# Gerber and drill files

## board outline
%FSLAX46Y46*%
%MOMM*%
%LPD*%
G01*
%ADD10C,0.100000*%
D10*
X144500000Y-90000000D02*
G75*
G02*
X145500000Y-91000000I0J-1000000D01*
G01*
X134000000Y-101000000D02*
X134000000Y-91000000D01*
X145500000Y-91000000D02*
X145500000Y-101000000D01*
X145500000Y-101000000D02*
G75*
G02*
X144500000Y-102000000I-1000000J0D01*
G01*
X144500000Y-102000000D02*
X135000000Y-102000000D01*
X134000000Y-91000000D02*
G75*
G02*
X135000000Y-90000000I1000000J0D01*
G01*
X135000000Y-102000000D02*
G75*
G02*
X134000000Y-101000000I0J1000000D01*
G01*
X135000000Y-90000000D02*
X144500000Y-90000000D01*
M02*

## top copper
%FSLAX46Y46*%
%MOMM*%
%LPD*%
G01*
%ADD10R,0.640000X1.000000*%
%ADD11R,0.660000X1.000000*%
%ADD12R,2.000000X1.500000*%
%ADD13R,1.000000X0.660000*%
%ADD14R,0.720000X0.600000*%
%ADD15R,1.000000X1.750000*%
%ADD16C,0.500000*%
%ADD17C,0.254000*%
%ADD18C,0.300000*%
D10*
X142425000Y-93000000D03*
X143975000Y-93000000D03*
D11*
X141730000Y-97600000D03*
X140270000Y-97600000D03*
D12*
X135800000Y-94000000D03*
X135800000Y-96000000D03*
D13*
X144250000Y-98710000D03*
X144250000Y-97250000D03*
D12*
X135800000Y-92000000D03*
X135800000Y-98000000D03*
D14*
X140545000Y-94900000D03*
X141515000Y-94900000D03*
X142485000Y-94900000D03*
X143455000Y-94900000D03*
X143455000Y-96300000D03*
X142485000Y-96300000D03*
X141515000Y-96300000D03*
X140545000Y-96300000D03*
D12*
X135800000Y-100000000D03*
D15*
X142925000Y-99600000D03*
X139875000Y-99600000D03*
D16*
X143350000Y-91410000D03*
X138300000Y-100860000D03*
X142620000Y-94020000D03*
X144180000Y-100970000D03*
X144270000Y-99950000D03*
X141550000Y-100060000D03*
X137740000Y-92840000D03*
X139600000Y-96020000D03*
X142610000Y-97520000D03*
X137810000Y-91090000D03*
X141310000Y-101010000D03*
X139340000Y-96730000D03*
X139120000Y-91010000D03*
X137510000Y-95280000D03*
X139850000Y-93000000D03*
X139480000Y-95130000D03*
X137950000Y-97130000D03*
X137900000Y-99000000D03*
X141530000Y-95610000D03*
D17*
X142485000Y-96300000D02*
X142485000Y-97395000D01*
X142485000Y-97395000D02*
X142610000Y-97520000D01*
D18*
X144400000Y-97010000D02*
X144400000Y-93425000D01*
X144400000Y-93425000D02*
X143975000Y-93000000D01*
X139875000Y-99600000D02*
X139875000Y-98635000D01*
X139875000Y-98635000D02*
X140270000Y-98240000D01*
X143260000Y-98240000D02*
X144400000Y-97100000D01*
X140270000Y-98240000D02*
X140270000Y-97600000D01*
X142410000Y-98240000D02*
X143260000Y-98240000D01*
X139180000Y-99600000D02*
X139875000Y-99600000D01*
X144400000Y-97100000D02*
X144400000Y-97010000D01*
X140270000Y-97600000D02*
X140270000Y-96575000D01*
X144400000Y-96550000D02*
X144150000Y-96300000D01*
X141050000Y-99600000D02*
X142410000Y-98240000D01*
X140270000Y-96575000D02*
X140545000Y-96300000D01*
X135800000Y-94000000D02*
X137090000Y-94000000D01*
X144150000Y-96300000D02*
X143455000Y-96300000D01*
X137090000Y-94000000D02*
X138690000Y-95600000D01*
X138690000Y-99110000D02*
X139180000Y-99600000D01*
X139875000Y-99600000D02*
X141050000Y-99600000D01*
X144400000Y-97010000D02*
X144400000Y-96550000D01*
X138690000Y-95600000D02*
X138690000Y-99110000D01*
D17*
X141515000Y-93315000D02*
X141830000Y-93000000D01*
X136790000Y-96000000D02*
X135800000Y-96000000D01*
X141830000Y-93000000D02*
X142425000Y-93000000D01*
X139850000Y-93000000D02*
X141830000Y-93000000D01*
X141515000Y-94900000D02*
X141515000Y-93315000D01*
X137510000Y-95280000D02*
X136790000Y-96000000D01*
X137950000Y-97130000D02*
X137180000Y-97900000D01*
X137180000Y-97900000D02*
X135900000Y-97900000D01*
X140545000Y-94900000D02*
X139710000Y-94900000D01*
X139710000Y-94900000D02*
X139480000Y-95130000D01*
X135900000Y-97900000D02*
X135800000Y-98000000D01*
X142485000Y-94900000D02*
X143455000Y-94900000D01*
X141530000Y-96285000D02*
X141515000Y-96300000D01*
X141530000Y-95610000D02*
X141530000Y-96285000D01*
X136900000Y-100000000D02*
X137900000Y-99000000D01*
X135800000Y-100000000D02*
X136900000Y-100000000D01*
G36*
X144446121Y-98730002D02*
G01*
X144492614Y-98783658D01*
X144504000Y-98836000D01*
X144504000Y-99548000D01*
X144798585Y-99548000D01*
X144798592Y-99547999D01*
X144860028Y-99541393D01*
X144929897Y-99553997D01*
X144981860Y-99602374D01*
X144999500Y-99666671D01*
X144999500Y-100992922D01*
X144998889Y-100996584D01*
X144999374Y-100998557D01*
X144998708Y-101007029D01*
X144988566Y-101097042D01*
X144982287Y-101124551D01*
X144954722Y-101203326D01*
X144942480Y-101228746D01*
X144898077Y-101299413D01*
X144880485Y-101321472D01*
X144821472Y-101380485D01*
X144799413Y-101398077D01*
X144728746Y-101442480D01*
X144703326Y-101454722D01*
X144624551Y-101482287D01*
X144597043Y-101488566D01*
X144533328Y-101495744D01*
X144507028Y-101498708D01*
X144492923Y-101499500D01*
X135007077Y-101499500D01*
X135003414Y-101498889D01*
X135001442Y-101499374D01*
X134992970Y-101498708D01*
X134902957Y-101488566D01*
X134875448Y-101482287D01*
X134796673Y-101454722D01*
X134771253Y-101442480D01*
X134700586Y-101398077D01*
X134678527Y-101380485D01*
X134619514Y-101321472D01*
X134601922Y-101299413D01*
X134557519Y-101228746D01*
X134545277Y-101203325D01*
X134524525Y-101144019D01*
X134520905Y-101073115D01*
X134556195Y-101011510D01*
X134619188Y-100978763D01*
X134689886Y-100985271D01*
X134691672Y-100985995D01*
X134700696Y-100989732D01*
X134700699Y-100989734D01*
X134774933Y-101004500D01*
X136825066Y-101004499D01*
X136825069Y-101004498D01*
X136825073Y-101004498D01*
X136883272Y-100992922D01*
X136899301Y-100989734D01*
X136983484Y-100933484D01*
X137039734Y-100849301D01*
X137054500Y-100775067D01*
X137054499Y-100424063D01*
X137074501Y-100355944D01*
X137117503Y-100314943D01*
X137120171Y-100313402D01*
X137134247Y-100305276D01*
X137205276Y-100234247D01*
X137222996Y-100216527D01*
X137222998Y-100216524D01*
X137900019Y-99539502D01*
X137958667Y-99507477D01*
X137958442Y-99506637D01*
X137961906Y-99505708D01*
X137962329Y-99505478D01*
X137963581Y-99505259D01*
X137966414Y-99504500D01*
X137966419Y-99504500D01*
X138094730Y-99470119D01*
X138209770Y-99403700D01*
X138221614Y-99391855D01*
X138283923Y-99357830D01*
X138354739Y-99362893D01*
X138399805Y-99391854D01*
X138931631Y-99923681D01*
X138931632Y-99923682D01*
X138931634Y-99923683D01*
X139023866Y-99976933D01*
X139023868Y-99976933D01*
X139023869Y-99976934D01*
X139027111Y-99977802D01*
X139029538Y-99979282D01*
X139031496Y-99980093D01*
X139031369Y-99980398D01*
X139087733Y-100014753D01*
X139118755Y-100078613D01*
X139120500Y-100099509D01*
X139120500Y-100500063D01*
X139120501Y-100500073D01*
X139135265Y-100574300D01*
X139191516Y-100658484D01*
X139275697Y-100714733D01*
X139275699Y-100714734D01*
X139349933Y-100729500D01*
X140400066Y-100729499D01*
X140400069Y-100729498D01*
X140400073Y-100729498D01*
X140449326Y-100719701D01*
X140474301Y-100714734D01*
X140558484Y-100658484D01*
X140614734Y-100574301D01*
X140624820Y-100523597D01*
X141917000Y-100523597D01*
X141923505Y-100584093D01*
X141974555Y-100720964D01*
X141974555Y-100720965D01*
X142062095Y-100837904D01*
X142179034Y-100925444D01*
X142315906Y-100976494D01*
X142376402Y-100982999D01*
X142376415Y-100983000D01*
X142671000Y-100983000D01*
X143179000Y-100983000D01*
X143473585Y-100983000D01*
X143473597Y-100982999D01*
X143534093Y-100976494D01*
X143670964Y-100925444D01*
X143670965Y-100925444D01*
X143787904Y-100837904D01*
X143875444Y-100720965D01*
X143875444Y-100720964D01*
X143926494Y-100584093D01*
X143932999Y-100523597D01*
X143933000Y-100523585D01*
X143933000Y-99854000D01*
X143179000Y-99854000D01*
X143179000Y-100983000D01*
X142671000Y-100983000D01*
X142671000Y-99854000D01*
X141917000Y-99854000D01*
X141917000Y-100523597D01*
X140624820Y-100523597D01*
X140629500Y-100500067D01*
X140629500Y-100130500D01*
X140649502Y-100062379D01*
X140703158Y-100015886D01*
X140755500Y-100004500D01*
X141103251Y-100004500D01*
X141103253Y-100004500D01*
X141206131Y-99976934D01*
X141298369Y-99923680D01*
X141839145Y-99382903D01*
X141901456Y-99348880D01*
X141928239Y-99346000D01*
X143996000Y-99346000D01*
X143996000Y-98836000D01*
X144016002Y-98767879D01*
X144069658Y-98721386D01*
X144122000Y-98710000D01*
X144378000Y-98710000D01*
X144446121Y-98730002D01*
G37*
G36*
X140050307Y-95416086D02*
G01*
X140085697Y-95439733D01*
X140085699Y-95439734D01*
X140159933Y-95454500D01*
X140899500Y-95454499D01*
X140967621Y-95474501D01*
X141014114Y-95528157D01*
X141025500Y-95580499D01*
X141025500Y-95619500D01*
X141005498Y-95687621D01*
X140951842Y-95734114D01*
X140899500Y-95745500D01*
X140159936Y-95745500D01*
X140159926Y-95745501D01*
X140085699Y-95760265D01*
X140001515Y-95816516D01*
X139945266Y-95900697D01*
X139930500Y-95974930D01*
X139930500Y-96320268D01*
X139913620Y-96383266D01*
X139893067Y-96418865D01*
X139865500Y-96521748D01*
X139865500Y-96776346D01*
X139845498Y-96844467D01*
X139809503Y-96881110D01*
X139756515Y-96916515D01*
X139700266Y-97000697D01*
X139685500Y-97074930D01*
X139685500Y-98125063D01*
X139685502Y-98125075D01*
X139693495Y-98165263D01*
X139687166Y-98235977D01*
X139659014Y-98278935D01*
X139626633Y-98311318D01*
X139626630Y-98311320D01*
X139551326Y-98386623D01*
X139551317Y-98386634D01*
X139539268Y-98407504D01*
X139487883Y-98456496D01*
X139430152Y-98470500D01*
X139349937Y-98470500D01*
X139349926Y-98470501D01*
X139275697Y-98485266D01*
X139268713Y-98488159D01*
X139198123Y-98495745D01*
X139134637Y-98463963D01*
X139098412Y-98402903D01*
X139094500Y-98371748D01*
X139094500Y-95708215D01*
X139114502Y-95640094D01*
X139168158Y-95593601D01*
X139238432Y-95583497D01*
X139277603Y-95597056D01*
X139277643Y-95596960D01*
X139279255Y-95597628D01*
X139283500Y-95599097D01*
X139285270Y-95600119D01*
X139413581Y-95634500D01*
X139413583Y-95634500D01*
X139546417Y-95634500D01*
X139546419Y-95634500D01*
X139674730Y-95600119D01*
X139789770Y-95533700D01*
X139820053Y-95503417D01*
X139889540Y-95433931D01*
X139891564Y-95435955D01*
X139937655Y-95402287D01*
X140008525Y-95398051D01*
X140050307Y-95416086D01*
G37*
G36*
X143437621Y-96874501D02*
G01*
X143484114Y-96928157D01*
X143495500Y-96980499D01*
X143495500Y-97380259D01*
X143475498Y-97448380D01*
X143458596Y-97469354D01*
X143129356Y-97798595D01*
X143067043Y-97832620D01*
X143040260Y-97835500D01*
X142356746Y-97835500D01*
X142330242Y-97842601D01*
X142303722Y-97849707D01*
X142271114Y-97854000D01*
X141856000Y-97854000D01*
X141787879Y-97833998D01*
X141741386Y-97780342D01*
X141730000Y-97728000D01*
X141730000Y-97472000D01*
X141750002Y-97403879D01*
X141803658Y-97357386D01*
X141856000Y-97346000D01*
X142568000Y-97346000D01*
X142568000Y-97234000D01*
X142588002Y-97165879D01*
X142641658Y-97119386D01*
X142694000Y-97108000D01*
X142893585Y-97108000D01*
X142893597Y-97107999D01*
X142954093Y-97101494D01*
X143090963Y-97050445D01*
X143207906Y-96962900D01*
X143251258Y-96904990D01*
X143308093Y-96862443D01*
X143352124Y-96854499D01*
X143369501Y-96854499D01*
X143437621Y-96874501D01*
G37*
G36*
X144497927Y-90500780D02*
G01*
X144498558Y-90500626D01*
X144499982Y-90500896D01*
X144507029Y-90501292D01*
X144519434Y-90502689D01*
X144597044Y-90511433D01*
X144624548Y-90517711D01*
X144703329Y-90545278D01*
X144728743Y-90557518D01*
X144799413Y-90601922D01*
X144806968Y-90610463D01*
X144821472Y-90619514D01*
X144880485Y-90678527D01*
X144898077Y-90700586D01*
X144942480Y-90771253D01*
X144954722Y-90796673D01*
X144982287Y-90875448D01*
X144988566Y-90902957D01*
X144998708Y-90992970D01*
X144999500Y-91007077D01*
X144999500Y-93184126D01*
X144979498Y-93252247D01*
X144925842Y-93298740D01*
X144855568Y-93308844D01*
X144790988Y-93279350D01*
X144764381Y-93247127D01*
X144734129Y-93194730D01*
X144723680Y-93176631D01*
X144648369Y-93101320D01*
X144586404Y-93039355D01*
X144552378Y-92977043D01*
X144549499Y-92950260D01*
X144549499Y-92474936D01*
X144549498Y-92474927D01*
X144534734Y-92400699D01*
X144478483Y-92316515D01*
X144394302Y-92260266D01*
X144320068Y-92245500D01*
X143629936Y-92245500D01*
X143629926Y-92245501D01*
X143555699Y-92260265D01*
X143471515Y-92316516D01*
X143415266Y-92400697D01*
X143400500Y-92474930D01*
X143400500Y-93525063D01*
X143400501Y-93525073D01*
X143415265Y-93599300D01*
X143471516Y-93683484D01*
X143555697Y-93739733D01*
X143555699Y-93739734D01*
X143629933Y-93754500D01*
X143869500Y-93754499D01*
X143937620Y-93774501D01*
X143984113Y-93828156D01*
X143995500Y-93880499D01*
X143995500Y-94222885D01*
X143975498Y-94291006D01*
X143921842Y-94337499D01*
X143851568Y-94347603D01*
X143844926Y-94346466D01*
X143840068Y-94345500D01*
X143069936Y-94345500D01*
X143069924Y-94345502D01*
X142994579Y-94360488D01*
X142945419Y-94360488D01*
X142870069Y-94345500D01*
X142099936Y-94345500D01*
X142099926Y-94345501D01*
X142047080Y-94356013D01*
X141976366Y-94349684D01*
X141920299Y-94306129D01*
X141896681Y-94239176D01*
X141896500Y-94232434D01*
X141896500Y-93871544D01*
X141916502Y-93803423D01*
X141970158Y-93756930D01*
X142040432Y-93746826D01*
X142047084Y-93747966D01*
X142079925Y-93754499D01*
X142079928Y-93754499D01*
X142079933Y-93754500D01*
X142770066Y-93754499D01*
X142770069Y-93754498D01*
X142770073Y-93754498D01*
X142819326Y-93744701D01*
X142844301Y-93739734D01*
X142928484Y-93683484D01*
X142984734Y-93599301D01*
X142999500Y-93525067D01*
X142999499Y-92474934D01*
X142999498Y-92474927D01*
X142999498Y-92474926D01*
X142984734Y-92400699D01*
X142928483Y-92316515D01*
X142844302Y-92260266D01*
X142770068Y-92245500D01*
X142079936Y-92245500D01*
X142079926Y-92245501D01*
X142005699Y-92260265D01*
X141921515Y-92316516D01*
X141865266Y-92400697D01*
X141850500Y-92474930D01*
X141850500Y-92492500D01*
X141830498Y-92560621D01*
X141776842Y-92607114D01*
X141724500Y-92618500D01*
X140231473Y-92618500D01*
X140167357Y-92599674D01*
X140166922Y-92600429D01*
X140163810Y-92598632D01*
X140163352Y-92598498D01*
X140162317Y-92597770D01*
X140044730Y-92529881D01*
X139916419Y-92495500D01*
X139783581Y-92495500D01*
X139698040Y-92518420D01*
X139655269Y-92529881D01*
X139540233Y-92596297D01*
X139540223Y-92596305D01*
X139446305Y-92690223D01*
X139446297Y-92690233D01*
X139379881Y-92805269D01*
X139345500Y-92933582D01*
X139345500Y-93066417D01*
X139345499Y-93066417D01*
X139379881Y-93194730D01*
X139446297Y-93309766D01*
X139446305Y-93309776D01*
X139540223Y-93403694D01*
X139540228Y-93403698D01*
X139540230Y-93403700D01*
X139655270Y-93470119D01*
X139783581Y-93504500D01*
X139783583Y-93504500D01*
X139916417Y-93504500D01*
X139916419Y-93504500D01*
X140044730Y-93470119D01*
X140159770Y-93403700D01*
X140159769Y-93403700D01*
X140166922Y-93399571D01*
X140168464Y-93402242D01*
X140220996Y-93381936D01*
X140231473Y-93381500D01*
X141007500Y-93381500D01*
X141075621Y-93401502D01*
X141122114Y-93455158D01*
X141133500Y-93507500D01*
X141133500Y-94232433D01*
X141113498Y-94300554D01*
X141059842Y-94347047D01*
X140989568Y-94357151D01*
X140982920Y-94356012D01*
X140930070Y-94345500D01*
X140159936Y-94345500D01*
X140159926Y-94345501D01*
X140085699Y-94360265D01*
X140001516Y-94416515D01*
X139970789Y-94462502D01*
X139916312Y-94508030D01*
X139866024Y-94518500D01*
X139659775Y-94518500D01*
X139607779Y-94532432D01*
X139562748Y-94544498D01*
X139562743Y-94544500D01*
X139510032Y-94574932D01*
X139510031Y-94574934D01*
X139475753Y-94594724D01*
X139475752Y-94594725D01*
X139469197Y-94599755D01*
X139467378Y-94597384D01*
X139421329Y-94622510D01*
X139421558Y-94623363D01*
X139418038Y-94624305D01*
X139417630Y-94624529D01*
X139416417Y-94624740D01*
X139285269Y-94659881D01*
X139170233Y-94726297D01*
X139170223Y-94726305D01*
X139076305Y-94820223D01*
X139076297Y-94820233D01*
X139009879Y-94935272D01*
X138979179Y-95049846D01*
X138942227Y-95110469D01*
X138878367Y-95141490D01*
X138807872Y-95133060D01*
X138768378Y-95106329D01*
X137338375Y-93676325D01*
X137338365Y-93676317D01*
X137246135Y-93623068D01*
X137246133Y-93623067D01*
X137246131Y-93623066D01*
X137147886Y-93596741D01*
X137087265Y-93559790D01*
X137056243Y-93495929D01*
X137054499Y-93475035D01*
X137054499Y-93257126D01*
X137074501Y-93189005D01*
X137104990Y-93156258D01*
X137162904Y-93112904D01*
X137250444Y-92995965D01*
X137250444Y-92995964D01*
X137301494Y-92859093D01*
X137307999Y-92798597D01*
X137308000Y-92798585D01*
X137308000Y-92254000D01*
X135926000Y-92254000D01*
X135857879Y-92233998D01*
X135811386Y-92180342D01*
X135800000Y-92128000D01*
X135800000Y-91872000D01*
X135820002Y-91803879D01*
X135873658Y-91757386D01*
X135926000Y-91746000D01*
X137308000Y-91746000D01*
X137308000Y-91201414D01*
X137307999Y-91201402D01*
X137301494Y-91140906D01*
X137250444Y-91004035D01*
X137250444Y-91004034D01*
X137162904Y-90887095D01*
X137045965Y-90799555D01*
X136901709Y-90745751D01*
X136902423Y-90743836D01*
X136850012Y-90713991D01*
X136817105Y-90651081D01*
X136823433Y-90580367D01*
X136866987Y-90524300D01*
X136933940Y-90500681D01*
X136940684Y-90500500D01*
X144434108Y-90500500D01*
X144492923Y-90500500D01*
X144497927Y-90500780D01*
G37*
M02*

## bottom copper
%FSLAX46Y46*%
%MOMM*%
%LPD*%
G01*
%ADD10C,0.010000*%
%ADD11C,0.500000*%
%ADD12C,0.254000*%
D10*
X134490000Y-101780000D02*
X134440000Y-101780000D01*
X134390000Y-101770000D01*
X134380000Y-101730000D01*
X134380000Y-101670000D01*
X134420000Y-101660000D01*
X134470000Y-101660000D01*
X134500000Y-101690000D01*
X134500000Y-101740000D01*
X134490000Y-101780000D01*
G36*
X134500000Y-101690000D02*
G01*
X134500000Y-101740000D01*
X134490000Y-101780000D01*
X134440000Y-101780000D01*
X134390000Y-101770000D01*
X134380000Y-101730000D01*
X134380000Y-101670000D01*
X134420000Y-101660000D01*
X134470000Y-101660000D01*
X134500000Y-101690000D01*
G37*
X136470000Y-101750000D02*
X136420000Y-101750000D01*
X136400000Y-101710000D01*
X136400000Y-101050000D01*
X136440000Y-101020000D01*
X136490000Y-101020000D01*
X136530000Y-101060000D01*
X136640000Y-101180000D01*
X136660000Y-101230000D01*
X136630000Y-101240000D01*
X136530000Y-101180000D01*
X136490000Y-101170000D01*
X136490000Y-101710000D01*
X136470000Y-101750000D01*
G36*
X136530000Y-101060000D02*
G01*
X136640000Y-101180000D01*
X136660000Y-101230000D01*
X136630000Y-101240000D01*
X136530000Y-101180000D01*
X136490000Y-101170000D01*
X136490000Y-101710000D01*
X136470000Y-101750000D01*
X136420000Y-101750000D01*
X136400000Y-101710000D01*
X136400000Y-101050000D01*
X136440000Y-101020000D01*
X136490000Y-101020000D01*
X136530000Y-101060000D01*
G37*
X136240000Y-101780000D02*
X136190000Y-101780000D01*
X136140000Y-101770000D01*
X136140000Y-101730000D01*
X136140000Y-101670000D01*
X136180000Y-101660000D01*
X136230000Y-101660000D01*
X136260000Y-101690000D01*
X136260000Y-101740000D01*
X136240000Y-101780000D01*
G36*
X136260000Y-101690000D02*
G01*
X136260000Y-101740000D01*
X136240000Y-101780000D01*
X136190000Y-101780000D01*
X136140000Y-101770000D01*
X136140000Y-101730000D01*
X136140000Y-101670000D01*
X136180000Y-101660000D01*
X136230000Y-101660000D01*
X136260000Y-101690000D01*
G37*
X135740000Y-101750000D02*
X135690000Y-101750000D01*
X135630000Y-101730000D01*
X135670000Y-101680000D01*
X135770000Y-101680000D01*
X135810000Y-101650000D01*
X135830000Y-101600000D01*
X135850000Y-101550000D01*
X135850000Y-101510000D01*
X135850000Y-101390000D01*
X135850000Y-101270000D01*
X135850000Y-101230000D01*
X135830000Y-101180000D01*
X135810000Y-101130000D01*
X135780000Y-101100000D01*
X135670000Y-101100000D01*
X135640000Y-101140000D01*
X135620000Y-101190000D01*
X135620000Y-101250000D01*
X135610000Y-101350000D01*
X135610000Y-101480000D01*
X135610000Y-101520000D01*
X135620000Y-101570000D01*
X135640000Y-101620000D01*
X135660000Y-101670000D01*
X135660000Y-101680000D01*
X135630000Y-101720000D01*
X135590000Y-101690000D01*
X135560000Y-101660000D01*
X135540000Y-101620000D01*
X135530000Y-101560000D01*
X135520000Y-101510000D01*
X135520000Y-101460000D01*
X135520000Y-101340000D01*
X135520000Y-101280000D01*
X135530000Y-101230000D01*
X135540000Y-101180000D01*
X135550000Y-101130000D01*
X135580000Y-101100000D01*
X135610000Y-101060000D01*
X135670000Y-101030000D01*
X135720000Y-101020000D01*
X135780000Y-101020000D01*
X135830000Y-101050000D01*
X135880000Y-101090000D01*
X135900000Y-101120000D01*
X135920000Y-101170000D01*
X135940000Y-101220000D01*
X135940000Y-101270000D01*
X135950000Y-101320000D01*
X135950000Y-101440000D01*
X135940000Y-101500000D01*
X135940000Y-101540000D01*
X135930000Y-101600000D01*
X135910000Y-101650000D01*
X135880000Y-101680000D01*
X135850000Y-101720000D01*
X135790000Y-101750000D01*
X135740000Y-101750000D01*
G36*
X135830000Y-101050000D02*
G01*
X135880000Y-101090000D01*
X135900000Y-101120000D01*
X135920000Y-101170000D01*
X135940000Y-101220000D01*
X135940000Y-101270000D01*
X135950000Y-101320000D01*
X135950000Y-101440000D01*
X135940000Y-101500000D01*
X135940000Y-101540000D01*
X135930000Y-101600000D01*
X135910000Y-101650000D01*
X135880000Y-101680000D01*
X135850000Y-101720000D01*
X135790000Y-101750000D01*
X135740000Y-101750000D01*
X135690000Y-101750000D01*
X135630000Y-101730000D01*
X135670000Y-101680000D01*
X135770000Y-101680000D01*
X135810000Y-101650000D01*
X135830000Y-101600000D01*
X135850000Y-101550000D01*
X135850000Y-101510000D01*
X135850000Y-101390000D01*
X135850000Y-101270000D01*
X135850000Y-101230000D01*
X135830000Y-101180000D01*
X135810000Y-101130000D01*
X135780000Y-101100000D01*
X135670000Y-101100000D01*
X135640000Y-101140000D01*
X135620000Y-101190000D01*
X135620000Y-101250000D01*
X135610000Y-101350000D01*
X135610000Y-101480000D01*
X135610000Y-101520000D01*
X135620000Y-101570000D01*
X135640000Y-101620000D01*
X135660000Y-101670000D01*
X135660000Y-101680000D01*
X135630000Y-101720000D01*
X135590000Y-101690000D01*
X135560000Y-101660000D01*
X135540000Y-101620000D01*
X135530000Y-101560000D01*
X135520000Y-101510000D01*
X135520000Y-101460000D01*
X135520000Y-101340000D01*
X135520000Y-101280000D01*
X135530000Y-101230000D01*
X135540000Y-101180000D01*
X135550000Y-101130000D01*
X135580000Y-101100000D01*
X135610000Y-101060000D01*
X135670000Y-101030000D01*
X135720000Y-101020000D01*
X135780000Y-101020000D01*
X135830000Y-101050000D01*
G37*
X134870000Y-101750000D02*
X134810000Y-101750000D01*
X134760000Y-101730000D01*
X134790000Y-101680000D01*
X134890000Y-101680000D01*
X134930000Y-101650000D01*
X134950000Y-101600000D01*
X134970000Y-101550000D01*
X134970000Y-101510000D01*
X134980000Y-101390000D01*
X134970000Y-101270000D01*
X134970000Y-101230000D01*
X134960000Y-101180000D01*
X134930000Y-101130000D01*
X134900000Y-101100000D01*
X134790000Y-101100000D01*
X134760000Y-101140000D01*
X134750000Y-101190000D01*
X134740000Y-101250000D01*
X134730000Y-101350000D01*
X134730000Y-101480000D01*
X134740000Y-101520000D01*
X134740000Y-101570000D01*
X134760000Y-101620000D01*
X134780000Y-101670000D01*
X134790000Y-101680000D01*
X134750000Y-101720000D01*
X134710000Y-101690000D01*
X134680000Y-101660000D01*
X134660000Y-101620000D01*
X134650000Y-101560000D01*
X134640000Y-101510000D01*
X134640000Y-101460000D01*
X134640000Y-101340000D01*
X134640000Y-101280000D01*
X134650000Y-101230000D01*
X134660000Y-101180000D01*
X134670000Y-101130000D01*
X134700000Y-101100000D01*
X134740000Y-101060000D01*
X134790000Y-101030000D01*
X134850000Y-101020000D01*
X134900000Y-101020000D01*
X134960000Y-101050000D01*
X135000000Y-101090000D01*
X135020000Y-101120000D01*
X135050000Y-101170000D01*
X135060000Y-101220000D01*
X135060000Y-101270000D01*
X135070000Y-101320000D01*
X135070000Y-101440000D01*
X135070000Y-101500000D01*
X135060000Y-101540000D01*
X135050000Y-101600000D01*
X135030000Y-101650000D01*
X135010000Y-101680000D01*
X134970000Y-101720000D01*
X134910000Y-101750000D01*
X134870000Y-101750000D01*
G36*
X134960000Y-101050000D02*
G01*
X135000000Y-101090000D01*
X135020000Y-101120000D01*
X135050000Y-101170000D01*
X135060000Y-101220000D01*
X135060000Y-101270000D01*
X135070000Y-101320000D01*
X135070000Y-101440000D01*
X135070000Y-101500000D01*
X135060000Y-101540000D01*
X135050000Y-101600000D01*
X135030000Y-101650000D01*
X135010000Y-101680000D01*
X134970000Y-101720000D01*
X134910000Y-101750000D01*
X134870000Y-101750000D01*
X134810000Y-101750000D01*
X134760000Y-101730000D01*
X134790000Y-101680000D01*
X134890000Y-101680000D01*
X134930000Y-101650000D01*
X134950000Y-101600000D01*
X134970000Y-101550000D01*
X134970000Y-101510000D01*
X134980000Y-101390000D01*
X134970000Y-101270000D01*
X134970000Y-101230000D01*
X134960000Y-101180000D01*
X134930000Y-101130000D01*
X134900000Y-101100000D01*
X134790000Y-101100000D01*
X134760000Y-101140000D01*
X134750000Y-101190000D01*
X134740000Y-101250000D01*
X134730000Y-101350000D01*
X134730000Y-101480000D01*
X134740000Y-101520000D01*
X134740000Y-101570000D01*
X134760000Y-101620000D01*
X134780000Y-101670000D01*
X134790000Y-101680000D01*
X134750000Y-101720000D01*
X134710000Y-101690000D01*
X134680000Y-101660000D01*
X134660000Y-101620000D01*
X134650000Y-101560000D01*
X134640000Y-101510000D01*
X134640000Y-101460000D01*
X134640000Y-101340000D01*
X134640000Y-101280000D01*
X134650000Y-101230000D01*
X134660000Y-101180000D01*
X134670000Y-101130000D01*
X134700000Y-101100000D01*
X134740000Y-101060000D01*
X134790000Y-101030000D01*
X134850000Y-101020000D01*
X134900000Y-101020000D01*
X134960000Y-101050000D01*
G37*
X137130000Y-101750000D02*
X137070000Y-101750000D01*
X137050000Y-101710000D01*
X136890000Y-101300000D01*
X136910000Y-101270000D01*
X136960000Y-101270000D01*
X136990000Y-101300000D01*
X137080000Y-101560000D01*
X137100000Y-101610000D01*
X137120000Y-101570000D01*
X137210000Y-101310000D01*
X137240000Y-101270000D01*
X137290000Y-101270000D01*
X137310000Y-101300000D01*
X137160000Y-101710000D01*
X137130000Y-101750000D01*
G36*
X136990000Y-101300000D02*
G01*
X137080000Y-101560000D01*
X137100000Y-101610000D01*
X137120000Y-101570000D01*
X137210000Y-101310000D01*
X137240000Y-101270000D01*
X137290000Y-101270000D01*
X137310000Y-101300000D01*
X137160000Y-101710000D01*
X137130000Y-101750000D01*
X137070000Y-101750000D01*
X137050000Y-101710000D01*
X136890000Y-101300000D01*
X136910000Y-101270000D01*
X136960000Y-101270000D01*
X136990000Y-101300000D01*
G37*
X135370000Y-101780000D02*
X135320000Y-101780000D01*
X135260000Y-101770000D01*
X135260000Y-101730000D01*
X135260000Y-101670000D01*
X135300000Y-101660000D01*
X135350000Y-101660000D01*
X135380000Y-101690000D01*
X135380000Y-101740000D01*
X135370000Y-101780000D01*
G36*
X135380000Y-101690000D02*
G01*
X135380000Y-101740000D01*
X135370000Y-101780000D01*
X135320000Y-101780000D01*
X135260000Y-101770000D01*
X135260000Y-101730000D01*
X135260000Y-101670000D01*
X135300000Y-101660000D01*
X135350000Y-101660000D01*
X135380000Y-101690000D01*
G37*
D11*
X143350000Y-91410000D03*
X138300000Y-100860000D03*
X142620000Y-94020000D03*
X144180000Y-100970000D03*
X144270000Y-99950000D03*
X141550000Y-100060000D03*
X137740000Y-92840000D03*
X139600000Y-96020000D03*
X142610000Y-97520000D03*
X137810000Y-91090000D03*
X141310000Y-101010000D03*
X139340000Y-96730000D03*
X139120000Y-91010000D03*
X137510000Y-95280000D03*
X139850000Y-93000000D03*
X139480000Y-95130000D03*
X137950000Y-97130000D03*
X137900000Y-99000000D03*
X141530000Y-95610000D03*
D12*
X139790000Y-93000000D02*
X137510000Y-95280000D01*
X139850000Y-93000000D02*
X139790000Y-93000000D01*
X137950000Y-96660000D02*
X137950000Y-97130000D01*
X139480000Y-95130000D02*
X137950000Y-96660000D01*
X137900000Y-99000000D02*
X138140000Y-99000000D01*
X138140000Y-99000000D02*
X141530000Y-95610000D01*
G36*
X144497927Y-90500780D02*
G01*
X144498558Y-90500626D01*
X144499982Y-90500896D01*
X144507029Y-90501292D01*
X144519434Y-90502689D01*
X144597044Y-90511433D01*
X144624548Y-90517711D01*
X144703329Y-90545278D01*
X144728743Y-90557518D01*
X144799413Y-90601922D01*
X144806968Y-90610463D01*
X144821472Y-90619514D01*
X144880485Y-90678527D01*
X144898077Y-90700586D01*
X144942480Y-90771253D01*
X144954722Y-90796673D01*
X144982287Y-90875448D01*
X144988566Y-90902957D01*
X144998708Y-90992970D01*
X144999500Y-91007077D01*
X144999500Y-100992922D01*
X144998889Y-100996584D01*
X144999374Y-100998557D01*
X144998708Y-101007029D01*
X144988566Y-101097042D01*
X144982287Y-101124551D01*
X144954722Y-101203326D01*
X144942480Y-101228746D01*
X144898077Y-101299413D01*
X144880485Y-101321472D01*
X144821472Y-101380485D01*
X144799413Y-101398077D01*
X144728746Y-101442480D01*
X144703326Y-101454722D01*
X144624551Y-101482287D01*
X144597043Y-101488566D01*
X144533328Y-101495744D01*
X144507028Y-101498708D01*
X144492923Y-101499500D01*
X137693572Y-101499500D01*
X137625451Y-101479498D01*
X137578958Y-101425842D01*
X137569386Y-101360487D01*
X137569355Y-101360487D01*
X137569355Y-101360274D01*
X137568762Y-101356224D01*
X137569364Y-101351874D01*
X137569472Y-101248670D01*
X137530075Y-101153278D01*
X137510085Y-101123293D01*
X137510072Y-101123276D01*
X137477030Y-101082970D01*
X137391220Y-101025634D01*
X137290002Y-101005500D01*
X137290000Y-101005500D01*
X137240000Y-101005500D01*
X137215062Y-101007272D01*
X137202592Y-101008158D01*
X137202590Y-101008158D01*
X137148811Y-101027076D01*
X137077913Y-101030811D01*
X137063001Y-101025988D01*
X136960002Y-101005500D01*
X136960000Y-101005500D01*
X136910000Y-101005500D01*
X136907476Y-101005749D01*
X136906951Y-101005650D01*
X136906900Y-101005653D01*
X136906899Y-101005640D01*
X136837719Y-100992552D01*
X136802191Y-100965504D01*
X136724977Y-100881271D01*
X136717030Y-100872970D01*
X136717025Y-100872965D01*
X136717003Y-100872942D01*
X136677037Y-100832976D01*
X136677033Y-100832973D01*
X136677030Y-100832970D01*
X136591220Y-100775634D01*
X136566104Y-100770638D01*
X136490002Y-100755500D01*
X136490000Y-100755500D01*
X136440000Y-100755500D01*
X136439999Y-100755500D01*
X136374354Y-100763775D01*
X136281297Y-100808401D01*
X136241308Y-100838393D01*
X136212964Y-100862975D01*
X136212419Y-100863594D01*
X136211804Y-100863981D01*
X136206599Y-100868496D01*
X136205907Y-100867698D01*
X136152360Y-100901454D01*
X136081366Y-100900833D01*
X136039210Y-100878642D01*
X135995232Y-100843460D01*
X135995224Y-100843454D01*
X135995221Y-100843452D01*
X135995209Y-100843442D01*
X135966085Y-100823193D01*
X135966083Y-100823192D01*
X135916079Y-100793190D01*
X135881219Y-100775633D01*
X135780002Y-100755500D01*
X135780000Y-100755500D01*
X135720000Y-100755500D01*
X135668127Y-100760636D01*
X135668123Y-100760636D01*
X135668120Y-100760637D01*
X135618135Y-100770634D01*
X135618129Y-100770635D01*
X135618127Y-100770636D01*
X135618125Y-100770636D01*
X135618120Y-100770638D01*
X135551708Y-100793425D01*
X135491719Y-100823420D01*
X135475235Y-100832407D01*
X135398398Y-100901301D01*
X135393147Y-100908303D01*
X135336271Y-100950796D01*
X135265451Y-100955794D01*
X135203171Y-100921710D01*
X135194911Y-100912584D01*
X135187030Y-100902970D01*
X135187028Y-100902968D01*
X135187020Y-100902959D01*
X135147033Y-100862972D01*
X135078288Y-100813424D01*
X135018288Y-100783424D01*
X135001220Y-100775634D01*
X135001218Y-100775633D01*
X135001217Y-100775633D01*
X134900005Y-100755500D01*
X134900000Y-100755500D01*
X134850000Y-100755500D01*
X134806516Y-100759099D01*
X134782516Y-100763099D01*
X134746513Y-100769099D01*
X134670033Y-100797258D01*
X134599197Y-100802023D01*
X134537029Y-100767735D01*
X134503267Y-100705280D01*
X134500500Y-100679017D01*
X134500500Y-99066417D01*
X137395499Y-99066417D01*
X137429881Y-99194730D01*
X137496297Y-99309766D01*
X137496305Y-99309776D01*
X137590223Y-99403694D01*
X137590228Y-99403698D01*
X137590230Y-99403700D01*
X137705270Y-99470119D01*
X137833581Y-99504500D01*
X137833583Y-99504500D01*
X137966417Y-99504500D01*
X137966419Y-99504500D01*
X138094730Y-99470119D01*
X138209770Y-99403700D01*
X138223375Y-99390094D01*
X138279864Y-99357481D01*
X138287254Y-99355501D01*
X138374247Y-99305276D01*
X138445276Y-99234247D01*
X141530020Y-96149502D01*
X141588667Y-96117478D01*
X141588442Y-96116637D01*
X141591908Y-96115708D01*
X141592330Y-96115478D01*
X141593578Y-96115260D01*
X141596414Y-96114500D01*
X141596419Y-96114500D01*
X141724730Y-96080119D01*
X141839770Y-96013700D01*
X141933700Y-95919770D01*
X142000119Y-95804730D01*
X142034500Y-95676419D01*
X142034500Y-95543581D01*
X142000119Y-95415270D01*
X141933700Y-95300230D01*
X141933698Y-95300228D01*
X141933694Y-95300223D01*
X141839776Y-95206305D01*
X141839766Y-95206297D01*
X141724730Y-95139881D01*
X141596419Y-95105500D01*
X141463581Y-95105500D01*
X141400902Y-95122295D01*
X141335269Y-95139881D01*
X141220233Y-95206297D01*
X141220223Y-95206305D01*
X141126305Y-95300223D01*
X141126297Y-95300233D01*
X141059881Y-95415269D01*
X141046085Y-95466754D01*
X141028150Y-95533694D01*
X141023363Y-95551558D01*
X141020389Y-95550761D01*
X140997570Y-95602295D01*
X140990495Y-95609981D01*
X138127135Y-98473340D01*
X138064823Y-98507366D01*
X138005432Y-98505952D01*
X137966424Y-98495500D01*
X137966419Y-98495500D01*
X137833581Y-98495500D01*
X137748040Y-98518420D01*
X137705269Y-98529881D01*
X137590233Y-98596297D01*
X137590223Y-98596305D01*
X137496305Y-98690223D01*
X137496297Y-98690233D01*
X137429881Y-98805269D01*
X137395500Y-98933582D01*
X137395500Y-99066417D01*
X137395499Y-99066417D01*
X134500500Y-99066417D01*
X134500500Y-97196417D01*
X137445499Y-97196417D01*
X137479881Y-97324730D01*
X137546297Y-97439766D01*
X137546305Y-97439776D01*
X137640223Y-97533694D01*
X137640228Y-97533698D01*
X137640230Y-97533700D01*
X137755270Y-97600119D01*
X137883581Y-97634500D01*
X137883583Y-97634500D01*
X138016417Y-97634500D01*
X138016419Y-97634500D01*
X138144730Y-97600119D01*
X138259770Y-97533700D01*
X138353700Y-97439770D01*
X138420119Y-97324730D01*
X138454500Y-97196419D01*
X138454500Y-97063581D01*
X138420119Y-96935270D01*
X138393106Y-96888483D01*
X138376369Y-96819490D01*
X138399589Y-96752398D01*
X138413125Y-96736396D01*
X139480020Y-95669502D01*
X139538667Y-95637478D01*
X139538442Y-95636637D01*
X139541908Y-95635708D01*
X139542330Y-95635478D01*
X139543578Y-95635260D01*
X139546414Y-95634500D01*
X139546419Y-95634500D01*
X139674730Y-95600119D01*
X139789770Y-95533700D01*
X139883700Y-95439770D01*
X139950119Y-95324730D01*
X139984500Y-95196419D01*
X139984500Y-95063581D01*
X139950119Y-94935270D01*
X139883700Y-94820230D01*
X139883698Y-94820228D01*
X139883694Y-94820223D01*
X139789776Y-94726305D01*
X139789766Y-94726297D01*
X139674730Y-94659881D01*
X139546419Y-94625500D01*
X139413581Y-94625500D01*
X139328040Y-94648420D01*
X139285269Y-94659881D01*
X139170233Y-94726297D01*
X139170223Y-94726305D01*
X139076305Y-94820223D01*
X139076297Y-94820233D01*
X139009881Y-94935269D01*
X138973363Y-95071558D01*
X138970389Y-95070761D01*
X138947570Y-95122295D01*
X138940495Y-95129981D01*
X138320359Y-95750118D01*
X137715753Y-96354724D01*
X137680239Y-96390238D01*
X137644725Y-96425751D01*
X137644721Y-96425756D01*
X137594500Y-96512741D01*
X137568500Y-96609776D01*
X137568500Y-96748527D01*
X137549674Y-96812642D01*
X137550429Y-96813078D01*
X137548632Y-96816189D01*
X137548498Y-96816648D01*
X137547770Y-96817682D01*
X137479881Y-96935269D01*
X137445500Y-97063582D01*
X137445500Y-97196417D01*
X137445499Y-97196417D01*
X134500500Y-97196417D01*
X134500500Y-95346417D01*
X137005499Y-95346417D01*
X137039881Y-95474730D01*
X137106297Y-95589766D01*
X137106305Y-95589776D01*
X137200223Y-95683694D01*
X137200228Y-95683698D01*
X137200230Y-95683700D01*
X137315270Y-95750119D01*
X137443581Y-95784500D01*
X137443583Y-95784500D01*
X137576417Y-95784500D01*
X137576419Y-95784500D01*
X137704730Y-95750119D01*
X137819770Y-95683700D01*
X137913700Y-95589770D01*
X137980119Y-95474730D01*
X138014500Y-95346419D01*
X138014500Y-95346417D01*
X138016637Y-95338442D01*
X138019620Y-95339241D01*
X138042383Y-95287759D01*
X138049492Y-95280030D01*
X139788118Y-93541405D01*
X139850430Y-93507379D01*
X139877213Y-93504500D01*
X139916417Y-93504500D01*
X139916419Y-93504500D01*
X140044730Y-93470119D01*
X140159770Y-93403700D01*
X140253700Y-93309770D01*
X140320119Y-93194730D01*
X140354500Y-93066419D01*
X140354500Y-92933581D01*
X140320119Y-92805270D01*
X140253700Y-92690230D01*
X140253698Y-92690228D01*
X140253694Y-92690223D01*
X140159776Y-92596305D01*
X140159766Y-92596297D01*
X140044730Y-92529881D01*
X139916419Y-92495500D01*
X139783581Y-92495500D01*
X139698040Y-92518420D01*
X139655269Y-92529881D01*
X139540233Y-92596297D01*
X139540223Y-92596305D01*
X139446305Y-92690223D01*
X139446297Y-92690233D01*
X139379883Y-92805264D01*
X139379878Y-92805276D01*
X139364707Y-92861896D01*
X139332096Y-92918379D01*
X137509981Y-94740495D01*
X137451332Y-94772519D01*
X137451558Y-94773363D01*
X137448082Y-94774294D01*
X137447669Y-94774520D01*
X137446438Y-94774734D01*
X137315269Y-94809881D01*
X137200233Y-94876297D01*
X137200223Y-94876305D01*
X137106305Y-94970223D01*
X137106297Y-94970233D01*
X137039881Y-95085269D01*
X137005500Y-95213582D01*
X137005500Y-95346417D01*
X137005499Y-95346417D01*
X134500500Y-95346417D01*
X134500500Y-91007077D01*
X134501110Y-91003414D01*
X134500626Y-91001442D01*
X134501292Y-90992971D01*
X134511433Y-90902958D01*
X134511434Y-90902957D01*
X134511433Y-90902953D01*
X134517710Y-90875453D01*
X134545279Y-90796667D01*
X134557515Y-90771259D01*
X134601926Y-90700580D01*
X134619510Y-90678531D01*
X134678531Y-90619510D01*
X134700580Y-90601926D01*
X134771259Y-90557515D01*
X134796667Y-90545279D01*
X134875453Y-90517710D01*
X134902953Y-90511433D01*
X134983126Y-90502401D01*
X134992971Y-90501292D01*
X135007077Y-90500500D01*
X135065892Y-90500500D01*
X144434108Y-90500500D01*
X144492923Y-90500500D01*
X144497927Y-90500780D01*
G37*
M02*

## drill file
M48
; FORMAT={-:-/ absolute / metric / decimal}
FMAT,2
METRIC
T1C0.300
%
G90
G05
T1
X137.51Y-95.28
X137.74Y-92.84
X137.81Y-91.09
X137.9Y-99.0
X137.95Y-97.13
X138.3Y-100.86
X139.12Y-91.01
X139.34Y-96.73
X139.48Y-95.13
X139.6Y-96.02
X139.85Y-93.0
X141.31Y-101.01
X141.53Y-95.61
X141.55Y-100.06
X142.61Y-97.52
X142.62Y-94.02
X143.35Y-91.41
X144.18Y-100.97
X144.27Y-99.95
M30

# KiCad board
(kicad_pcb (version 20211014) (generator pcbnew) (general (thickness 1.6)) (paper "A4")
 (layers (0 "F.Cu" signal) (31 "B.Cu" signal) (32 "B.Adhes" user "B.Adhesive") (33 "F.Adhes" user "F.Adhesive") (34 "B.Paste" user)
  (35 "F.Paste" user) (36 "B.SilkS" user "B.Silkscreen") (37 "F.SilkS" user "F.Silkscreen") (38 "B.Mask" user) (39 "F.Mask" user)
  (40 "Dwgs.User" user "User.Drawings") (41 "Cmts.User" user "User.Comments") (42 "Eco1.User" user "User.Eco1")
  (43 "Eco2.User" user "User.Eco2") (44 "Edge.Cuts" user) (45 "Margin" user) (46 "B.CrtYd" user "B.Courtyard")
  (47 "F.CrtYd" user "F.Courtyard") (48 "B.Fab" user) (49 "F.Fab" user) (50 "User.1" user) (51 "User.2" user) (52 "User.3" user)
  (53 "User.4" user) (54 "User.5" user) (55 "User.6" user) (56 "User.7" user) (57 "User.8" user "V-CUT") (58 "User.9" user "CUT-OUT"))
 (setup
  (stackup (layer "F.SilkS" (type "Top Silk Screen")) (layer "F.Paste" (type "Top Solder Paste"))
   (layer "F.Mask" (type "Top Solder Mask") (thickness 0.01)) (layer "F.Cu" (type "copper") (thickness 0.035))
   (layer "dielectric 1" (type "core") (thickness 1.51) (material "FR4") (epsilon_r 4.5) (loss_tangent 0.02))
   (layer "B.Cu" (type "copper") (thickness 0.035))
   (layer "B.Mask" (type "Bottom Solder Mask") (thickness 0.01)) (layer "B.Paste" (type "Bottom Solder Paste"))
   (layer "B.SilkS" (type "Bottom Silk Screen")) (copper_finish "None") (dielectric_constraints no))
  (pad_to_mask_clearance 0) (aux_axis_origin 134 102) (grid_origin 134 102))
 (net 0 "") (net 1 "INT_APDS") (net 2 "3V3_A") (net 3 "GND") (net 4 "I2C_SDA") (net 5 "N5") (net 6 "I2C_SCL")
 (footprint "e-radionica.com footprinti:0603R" (layer "F.Cu") (at 143.2 93)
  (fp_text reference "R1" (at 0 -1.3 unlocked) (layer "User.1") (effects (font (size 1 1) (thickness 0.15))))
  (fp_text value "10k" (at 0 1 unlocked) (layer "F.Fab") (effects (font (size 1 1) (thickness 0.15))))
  (pad "1" smd rect locked (at -0.775 0 90) (size 1 0.64) (layers "F.Cu" "F.Paste" "F.Mask") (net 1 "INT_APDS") (solder_mask_margin 0.1))
  (pad "2" smd rect locked (at 0.775 0 90) (size 1 0.64) (layers "F.Cu" "F.Paste" "F.Mask") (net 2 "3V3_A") (solder_mask_margin 0.1)))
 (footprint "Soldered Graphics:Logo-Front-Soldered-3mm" (layer "F.Cu") (at 140.84 91.64)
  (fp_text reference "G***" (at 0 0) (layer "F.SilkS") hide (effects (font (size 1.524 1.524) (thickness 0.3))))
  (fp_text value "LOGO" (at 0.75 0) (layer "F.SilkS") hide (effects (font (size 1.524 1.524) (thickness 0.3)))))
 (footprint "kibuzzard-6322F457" (layer "F.Cu") (at 138.2 96)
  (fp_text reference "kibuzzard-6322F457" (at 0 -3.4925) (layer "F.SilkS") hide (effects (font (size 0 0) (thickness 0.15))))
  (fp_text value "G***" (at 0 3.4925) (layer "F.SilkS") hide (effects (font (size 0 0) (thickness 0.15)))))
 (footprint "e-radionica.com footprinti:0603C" (layer "F.Cu") (at 141 97.6 180)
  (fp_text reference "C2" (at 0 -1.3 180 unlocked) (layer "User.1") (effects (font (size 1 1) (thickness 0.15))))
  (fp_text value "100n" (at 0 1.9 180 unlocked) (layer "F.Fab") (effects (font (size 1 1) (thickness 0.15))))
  (pad "1" smd rect locked (at -0.73 0 180) (size 0.66 1) (layers "F.Cu" "F.Paste" "F.Mask") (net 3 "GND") (solder_mask_margin 0.1))
  (pad "2" smd rect locked (at 0.73 0 180) (size 0.66 1) (layers "F.Cu" "F.Paste" "F.Mask") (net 2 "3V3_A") (solder_mask_margin 0.1)))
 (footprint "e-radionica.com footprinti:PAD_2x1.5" (layer "F.Cu") (at 135.8 94)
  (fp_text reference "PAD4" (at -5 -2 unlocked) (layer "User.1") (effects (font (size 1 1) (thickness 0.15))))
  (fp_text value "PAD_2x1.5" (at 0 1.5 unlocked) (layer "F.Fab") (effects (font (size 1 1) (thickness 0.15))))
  (pad "1" smd rect (at 0 0) (size 2 1.5) (layers "F.Cu" "F.Paste" "F.Mask") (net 2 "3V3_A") (solder_mask_margin 0.1)))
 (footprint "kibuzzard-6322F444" (layer "F.Cu") (at 138.2 92)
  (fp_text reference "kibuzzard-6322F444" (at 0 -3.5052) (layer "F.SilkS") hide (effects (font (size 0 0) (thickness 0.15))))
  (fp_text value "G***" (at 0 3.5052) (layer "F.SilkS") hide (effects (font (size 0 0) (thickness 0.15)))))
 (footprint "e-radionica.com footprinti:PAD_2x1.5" (layer "F.Cu") (at 135.8 96)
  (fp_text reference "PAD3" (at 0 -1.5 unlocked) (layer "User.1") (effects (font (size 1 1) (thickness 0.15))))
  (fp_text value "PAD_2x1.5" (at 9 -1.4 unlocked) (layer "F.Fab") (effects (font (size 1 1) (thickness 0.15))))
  (pad "1" smd rect (at 0 0) (size 2 1.5) (layers "F.Cu" "F.Paste" "F.Mask") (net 1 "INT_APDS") (solder_mask_margin 0.1)))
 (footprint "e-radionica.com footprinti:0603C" (layer "F.Cu") (at 144.25 97.98 90)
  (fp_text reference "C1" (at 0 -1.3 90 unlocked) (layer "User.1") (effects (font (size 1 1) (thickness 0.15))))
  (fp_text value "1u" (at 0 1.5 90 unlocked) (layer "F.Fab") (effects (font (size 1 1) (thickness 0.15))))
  (pad "1" smd rect locked (at -0.73 0 90) (size 0.66 1) (layers "F.Cu" "F.Paste" "F.Mask") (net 3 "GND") (solder_mask_margin 0.1))
  (pad "2" smd rect locked (at 0.73 0 90) (size 0.66 1) (layers "F.Cu" "F.Paste" "F.Mask") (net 2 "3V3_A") (solder_mask_margin 0.1)))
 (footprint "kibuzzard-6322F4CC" (layer "F.Cu") (at 138.2 98)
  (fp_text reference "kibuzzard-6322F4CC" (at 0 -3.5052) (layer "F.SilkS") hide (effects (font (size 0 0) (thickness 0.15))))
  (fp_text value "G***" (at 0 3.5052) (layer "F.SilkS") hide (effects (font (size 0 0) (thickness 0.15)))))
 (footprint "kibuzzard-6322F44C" (layer "F.Cu") (at 138.2 94)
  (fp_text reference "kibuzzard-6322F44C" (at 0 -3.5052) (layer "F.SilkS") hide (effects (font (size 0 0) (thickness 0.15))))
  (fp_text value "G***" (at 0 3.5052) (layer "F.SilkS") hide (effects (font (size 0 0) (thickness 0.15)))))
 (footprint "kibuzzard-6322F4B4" (layer "F.Cu") (at 138.2 100)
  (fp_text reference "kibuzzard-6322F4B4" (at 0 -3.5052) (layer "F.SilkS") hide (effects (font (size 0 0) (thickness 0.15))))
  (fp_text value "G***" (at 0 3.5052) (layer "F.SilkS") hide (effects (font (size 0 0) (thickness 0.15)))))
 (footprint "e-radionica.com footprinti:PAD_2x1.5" (layer "F.Cu") (at 135.8 92)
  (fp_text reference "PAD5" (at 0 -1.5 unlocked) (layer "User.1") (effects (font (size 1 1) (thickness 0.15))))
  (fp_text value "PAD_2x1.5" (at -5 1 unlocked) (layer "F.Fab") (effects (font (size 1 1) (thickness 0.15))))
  (pad "1" smd rect (at 0 0) (size 2 1.5) (layers "F.Cu" "F.Paste" "F.Mask") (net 3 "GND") (solder_mask_margin 0.1)))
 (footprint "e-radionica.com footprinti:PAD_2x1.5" (layer "F.Cu") (at 135.8 98)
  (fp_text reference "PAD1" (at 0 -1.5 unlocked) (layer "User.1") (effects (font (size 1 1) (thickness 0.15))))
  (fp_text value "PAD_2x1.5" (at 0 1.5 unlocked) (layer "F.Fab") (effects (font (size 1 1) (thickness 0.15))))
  (pad "1" smd rect (at 0 0) (size 2 1.5) (layers "F.Cu" "F.Paste" "F.Mask") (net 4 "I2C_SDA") (solder_mask_margin 0.1)))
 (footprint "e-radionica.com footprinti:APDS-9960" (layer "F.Cu") (at 142 95.6 90)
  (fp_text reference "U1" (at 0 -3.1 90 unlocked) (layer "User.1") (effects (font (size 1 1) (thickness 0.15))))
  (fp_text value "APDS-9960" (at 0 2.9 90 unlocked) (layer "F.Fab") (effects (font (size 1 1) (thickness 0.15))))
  (pad "1" smd rect (at 0.7 -1.455 90) (size 0.6 0.72) (layers "F.Cu" "F.Paste" "F.Mask") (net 4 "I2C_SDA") (solder_mask_margin 0.1))
  (pad "2" smd rect (at 0.7 -0.485 90) (size 0.6 0.72) (layers "F.Cu" "F.Paste" "F.Mask") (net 1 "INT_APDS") (solder_mask_margin 0.1))
  (pad "3" smd rect (at 0.7 0.485 90) (size 0.6 0.72) (layers "F.Cu" "F.Paste" "F.Mask") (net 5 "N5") (solder_mask_margin 0.1))
  (pad "4" smd rect (at 0.7 1.455 90) (size 0.6 0.72) (layers "F.Cu" "F.Paste" "F.Mask") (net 5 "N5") (solder_mask_margin 0.1))
  (pad "5" smd rect (at -0.7 1.455 90) (size 0.6 0.72) (layers "F.Cu" "F.Paste" "F.Mask") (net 2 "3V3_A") (solder_mask_margin 0.1))
  (pad "6" smd rect (at -0.7 0.485 90) (size 0.6 0.72) (layers "F.Cu" "F.Paste" "F.Mask") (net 3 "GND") (solder_mask_margin 0.1))
  (pad "7" smd rect (at -0.7 -0.485 90) (size 0.6 0.72) (layers "F.Cu" "F.Paste" "F.Mask") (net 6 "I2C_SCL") (solder_mask_margin 0.1))
  (pad "8" smd rect (at -0.7 -1.455 90) (size 0.6 0.72) (layers "F.Cu" "F.Paste" "F.Mask") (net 2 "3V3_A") (solder_mask_margin 0.1)))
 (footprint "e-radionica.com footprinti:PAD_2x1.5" (layer "F.Cu") (at 135.8 100)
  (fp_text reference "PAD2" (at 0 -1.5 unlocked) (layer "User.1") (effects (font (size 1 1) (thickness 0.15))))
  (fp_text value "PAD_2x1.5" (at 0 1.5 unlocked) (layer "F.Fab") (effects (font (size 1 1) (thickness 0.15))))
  (pad "1" smd rect (at 0 0) (size 2 1.5) (layers "F.Cu" "F.Paste" "F.Mask") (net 6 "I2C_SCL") (solder_mask_margin 0.1)))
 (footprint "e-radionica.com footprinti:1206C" (layer "F.Cu") (at 141.4 99.6 180)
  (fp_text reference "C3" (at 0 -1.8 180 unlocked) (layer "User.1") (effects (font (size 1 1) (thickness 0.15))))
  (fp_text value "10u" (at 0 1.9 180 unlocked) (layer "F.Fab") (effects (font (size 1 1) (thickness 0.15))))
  (pad "1" smd rect locked (at -1.525 0 270) (size 1.75 1) (layers "F.Cu" "F.Paste" "F.Mask") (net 3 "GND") (solder_mask_margin 0.1))
  (pad "2" smd rect locked (at 1.525 0 270) (size 1.75 1) (layers "F.Cu" "F.Paste" "F.Mask") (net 2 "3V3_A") (solder_mask_margin 0.1)))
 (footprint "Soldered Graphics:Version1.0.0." (layer "B.Cu") (at 135.8 101.4 180)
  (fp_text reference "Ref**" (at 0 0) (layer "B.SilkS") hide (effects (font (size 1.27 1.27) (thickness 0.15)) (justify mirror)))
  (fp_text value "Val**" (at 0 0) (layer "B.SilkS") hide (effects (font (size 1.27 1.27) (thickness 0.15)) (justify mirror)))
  (fp_poly
   (pts (xy 1.31 -0.38) (xy 1.36 -0.38) (xy 1.41 -0.37) (xy 1.42 -0.33) (xy 1.42 -0.27) (xy 1.38 -0.26) (xy 1.33 -0.26) (xy 1.3 -0.29)
    (xy 1.3 -0.34) (xy 1.31 -0.38))
   (layer "B.Cu") (width 0.01) (fill solid))
  (fp_poly
   (pts (xy -0.67 -0.35) (xy -0.62 -0.35) (xy -0.6 -0.31) (xy -0.6 0.35) (xy -0.64 0.38) (xy -0.69 0.38) (xy -0.73 0.34) (xy -0.84 0.22)
    (xy -0.86 0.17) (xy -0.83 0.16) (xy -0.73 0.22) (xy -0.69 0.23) (xy -0.69 -0.31) (xy -0.67 -0.35))
   (layer "B.Cu") (width 0.01) (fill solid))
  (fp_poly
   (pts (xy -0.44 -0.38) (xy -0.39 -0.38) (xy -0.34 -0.37) (xy -0.34 -0.33) (xy -0.34 -0.27) (xy -0.38 -0.26) (xy -0.43 -0.26)
    (xy -0.46 -0.29) (xy -0.46 -0.34) (xy -0.44 -0.38))
   (layer "B.Cu") (width 0.01) (fill solid))
  (fp_poly
   (pts (xy 0.06 -0.35) (xy 0.11 -0.35) (xy 0.17 -0.33) (xy 0.13 -0.28) (xy 0.03 -0.28) (xy -0.01 -0.25) (xy -0.03 -0.2) (xy -0.05 -0.15)
    (xy -0.05 -0.11) (xy -0.05 0.01) (xy -0.05 0.13) (xy -0.05 0.17) (xy -0.03 0.22) (xy -0.01 0.27) (xy 0.02 0.3) (xy 0.13 0.3)
    (xy 0.16 0.26) (xy 0.18 0.21) (xy 0.18 0.15) (xy 0.19 0.05) (xy 0.19 -0.08) (xy 0.19 -0.12) (xy 0.18 -0.17) (xy 0.16 -0.22)
    (xy 0.14 -0.27) (xy 0.14 -0.28) (xy 0.17 -0.32) (xy 0.21 -0.29) (xy 0.24 -0.26) (xy 0.26 -0.22) (xy 0.27 -0.16) (xy 0.28 -0.11)
    (xy 0.28 -0.06) (xy 0.28 0.06) (xy 0.28 0.12) (xy 0.27 0.17) (xy 0.26 0.22) (xy 0.25 0.27) (xy 0.22 0.3) (xy 0.19 0.34) (xy 0.13 0.37)
    (xy 0.08 0.38) (xy 0.02 0.38) (xy -0.03 0.35) (xy -0.08 0.31) (xy -0.1 0.28) (xy -0.12 0.23) (xy -0.14 0.18) (xy -0.14 0.13)
    (xy -0.15 0.08) (xy -0.15 -0.04) (xy -0.14 -0.1) (xy -0.14 -0.14) (xy -0.13 -0.2) (xy -0.11 -0.25) (xy -0.08 -0.28) (xy -0.05 -0.32)
    (xy 0.01 -0.35) (xy 0.06 -0.35))
   (layer "B.Cu") (width 0.01) (fill solid))
  (fp_poly
   (pts (xy 0.93 -0.35) (xy 0.99 -0.35) (xy 1.04 -0.33) (xy 1.01 -0.28) (xy 0.91 -0.28) (xy 0.87 -0.25) (xy 0.85 -0.2) (xy 0.83 -0.15)
    (xy 0.83 -0.11) (xy 0.82 0.01) (xy 0.83 0.13) (xy 0.83 0.17) (xy 0.84 0.22) (xy 0.87 0.27) (xy 0.9 0.3) (xy 1.01 0.3) (xy 1.04 0.26)
    (xy 1.05 0.21) (xy 1.06 0.15) (xy 1.07 0.05) (xy 1.07 -0.08) (xy 1.06 -0.12) (xy 1.06 -0.17) (xy 1.04 -0.22) (xy 1.02 -0.27)
    (xy 1.01 -0.28) (xy 1.05 -0.32) (xy 1.09 -0.29) (xy 1.12 -0.26) (xy 1.14 -0.22) (xy 1.15 -0.16) (xy 1.16 -0.11) (xy 1.16 -0.06)
    (xy 1.16 0.06) (xy 1.16 0.12) (xy 1.15 0.17) (xy 1.14 0.22) (xy 1.13 0.27) (xy 1.1 0.3) (xy 1.06 0.34) (xy 1.01 0.37) (xy 0.95 0.38)
    (xy 0.9 0.38) (xy 0.84 0.35) (xy 0.8 0.31) (xy 0.78 0.28) (xy 0.75 0.23) (xy 0.74 0.18) (xy 0.74 0.13) (xy 0.73 0.08) (xy 0.73 -0.04)
    (xy 0.73 -0.1) (xy 0.74 -0.14) (xy 0.75 -0.2) (xy 0.77 -0.25) (xy 0.79 -0.28) (xy 0.83 -0.32) (xy 0.89 -0.35) (xy 0.93 -0.35))
   (layer "B.Cu") (width 0.01) (fill solid))
  (fp_poly
   (pts (xy -1.33 -0.35) (xy -1.27 -0.35) (xy -1.25 -0.31) (xy -1.09 0.1) (xy -1.11 0.13) (xy -1.16 0.13) (xy -1.19 0.1) (xy -1.28 -0.16)
    (xy -1.3 -0.21) (xy -1.32 -0.17) (xy -1.41 0.09) (xy -1.44 0.13) (xy -1.49 0.13) (xy -1.51 0.1) (xy -1.36 -0.31) (xy -1.33 -0.35))
   (layer "B.Cu") (width 0.01) (fill solid))
  (fp_poly
   (pts (xy 0.43 -0.38) (xy 0.48 -0.38) (xy 0.54 -0.37) (xy 0.54 -0.33) (xy 0.54 -0.27) (xy 0.5 -0.26) (xy 0.45 -0.26) (xy 0.42 -0.29)
    (xy 0.42 -0.34) (xy 0.43 -0.38))
   (layer "B.Cu") (width 0.01) (fill solid)))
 (gr_arc (start 144.5 90) (mid 145.207107 90.292893) (end 145.5 91) (layer "Edge.Cuts") (width 0.1))
 (gr_line (start 134 101) (end 134 91) (layer "Edge.Cuts") (width 0.1))
 (gr_line (start 145.5 91) (end 145.5 101) (layer "Edge.Cuts") (width 0.1))
 (gr_arc (start 145.5 101) (mid 145.207107 101.707107) (end 144.5 102) (layer "Edge.Cuts") (width 0.1))
 (gr_line (start 144.5 102) (end 135 102) (layer "Edge.Cuts") (width 0.1))
 (gr_arc (start 134 91) (mid 134.292893 90.292893) (end 135 90) (layer "Edge.Cuts") (width 0.1))
 (gr_arc (start 135 102) (mid 134.292893 101.707107) (end 134 101) (layer "Edge.Cuts") (width 0.1))
 (gr_line (start 135 90) (end 144.5 90) (layer "Edge.Cuts") (width 0.1))
 (segment (start 142.485 96.3) (end 142.485 97.395) (width 0.254) (layer "F.Cu") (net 3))
 (segment (start 142.485 97.395) (end 142.61 97.52) (width 0.254) (layer "F.Cu") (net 3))
 (via (at 143.35 91.41) (size 0.5) (drill 0.3) (layers "F.Cu" "B.Cu") (free) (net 3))
 (via (at 138.3 100.86) (size 0.5) (drill 0.3) (layers "F.Cu" "B.Cu") (free) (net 3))
 (via (at 142.62 94.02) (size 0.5) (drill 0.3) (layers "F.Cu" "B.Cu") (free) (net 3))
 (via (at 144.18 100.97) (size 0.5) (drill 0.3) (layers "F.Cu" "B.Cu") (free) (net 3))
 (via (at 144.27 99.95) (size 0.5) (drill 0.3) (layers "F.Cu" "B.Cu") (free) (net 3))
 (via (at 141.55 100.06) (size 0.5) (drill 0.3) (layers "F.Cu" "B.Cu") (free) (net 3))
 (via (at 137.74 92.84) (size 0.5) (drill 0.3) (layers "F.Cu" "B.Cu") (free) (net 3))
 (via (at 139.6 96.02) (size 0.5) (drill 0.3) (layers "F.Cu" "B.Cu") (free) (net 3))
 (via (at 142.61 97.52) (size 0.5) (drill 0.3) (layers "F.Cu" "B.Cu") (free) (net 3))
 (via (at 137.81 91.09) (size 0.5) (drill 0.3) (layers "F.Cu" "B.Cu") (free) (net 3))
 (via (at 141.31 101.01) (size 0.5) (drill 0.3) (layers "F.Cu" "B.Cu") (free) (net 3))
 (via (at 139.34 96.73) (size 0.5) (drill 0.3) (layers "F.Cu" "B.Cu") (free) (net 3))
 (via (at 139.12 91.01) (size 0.5) (drill 0.3) (layers "F.Cu" "B.Cu") (free) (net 3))
 (segment (start 144.4 97.01) (end 144.4 93.425) (width 0.3) (layer "F.Cu") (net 2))
 (segment (start 144.4 93.425) (end 143.975 93) (width 0.3) (layer "F.Cu") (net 2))
 (segment (start 139.875 99.6) (end 139.875 98.635) (width 0.3) (layer "F.Cu") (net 2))
 (segment (start 139.875 98.635) (end 140.27 98.24) (width 0.3) (layer "F.Cu") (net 2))
 (segment (start 143.26 98.24) (end 144.4 97.1) (width 0.3) (layer "F.Cu") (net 2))
 (segment (start 140.27 98.24) (end 140.27 97.6) (width 0.3) (layer "F.Cu") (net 2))
 (segment (start 142.41 98.24) (end 143.26 98.24) (width 0.3) (layer "F.Cu") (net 2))
 (segment (start 139.18 99.6) (end 139.875 99.6) (width 0.3) (layer "F.Cu") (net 2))
 (segment (start 144.4 97.1) (end 144.4 97.01) (width 0.3) (layer "F.Cu") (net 2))
 (segment (start 140.27 97.6) (end 140.27 96.575) (width 0.3) (layer "F.Cu") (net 2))
 (segment (start 144.4 96.55) (end 144.15 96.3) (width 0.3) (layer "F.Cu") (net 2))
 (segment (start 141.05 99.6) (end 142.41 98.24) (width 0.3) (layer "F.Cu") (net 2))
 (segment (start 140.27 96.575) (end 140.545 96.3) (width 0.3) (layer "F.Cu") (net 2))
 (segment (start 135.8 94) (end 137.09 94) (width 0.3) (layer "F.Cu") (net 2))
 (segment (start 144.15 96.3) (end 143.455 96.3) (width 0.3) (layer "F.Cu") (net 2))
 (segment (start 137.09 94) (end 138.69 95.6) (width 0.3) (layer "F.Cu") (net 2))
 (segment (start 138.69 99.11) (end 139.18 99.6) (width 0.3) (layer "F.Cu") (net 2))
 (segment (start 139.875 99.6) (end 141.05 99.6) (width 0.3) (layer "F.Cu") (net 2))
 (segment (start 144.4 97.01) (end 144.4 96.55) (width 0.3) (layer "F.Cu") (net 2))
 (segment (start 138.69 95.6) (end 138.69 99.11) (width 0.3) (layer "F.Cu") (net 2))
 (segment (start 141.515 93.315) (end 141.83 93) (width 0.254) (layer "F.Cu") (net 1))
 (segment (start 136.79 96) (end 135.8 96) (width 0.254) (layer "F.Cu") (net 1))
 (segment (start 141.83 93) (end 142.425 93) (width 0.254) (layer "F.Cu") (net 1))
 (segment (start 139.85 93) (end 141.83 93) (width 0.254) (layer "F.Cu") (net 1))
 (segment (start 141.515 94.9) (end 141.515 93.315) (width 0.254) (layer "F.Cu") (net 1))
 (segment (start 137.51 95.28) (end 136.79 96) (width 0.254) (layer "F.Cu") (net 1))
 (via (at 137.51 95.28) (size 0.5) (drill 0.3) (layers "F.Cu" "B.Cu") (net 1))
 (via (at 139.85 93) (size 0.5) (drill 0.3) (layers "F.Cu" "B.Cu") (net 1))
 (segment (start 139.79 93) (end 137.51 95.28) (width 0.254) (layer "B.Cu") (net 1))
 (segment (start 139.85 93) (end 139.79 93) (width 0.254) (layer "B.Cu") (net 1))
 (segment (start 137.95 97.13) (end 137.18 97.9) (width 0.254) (layer "F.Cu") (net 4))
 (segment (start 137.18 97.9) (end 135.9 97.9) (width 0.254) (layer "F.Cu") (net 4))
 (segment (start 140.545 94.9) (end 139.71 94.9) (width 0.254) (layer "F.Cu") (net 4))
 (segment (start 139.71 94.9) (end 139.48 95.13) (width 0.254) (layer "F.Cu") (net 4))
 (segment (start 135.9 97.9) (end 135.8 98) (width 0.254) (layer "F.Cu") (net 4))
 (via (at 139.48 95.13) (size 0.5) (drill 0.3) (layers "F.Cu" "B.Cu") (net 4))
 (via (at 137.95 97.13) (size 0.5) (drill 0.3) (layers "F.Cu" "B.Cu") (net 4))
 (segment (start 137.95 96.66) (end 137.95 97.13) (width 0.254) (layer "B.Cu") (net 4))
 (segment (start 139.48 95.13) (end 137.95 96.66) (width 0.254) (layer "B.Cu") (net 4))
 (segment (start 142.485 94.9) (end 143.455 94.9) (width 0.254) (layer "F.Cu") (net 5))
 (segment (start 141.53 96.285) (end 141.515 96.3) (width 0.254) (layer "F.Cu") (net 6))
 (segment (start 141.53 95.61) (end 141.53 96.285) (width 0.254) (layer "F.Cu") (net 6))
 (segment (start 136.9 100) (end 137.9 99) (width 0.254) (layer "F.Cu") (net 6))
 (segment (start 135.8 100) (end 136.9 100) (width 0.254) (layer "F.Cu") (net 6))
 (via (at 137.9 99) (size 0.5) (drill 0.3) (layers "F.Cu" "B.Cu") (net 6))
 (via (at 141.53 95.61) (size 0.5) (drill 0.3) (layers "F.Cu" "B.Cu") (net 6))
 (segment (start 137.9 99) (end 138.14 99) (width 0.254) (layer "B.Cu") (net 6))
 (segment (start 138.14 99) (end 141.53 95.61) (width 0.254) (layer "B.Cu") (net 6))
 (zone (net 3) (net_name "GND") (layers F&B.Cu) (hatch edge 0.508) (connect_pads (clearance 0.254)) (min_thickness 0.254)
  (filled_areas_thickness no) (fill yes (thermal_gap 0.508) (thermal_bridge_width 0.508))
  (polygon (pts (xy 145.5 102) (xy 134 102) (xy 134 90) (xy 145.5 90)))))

